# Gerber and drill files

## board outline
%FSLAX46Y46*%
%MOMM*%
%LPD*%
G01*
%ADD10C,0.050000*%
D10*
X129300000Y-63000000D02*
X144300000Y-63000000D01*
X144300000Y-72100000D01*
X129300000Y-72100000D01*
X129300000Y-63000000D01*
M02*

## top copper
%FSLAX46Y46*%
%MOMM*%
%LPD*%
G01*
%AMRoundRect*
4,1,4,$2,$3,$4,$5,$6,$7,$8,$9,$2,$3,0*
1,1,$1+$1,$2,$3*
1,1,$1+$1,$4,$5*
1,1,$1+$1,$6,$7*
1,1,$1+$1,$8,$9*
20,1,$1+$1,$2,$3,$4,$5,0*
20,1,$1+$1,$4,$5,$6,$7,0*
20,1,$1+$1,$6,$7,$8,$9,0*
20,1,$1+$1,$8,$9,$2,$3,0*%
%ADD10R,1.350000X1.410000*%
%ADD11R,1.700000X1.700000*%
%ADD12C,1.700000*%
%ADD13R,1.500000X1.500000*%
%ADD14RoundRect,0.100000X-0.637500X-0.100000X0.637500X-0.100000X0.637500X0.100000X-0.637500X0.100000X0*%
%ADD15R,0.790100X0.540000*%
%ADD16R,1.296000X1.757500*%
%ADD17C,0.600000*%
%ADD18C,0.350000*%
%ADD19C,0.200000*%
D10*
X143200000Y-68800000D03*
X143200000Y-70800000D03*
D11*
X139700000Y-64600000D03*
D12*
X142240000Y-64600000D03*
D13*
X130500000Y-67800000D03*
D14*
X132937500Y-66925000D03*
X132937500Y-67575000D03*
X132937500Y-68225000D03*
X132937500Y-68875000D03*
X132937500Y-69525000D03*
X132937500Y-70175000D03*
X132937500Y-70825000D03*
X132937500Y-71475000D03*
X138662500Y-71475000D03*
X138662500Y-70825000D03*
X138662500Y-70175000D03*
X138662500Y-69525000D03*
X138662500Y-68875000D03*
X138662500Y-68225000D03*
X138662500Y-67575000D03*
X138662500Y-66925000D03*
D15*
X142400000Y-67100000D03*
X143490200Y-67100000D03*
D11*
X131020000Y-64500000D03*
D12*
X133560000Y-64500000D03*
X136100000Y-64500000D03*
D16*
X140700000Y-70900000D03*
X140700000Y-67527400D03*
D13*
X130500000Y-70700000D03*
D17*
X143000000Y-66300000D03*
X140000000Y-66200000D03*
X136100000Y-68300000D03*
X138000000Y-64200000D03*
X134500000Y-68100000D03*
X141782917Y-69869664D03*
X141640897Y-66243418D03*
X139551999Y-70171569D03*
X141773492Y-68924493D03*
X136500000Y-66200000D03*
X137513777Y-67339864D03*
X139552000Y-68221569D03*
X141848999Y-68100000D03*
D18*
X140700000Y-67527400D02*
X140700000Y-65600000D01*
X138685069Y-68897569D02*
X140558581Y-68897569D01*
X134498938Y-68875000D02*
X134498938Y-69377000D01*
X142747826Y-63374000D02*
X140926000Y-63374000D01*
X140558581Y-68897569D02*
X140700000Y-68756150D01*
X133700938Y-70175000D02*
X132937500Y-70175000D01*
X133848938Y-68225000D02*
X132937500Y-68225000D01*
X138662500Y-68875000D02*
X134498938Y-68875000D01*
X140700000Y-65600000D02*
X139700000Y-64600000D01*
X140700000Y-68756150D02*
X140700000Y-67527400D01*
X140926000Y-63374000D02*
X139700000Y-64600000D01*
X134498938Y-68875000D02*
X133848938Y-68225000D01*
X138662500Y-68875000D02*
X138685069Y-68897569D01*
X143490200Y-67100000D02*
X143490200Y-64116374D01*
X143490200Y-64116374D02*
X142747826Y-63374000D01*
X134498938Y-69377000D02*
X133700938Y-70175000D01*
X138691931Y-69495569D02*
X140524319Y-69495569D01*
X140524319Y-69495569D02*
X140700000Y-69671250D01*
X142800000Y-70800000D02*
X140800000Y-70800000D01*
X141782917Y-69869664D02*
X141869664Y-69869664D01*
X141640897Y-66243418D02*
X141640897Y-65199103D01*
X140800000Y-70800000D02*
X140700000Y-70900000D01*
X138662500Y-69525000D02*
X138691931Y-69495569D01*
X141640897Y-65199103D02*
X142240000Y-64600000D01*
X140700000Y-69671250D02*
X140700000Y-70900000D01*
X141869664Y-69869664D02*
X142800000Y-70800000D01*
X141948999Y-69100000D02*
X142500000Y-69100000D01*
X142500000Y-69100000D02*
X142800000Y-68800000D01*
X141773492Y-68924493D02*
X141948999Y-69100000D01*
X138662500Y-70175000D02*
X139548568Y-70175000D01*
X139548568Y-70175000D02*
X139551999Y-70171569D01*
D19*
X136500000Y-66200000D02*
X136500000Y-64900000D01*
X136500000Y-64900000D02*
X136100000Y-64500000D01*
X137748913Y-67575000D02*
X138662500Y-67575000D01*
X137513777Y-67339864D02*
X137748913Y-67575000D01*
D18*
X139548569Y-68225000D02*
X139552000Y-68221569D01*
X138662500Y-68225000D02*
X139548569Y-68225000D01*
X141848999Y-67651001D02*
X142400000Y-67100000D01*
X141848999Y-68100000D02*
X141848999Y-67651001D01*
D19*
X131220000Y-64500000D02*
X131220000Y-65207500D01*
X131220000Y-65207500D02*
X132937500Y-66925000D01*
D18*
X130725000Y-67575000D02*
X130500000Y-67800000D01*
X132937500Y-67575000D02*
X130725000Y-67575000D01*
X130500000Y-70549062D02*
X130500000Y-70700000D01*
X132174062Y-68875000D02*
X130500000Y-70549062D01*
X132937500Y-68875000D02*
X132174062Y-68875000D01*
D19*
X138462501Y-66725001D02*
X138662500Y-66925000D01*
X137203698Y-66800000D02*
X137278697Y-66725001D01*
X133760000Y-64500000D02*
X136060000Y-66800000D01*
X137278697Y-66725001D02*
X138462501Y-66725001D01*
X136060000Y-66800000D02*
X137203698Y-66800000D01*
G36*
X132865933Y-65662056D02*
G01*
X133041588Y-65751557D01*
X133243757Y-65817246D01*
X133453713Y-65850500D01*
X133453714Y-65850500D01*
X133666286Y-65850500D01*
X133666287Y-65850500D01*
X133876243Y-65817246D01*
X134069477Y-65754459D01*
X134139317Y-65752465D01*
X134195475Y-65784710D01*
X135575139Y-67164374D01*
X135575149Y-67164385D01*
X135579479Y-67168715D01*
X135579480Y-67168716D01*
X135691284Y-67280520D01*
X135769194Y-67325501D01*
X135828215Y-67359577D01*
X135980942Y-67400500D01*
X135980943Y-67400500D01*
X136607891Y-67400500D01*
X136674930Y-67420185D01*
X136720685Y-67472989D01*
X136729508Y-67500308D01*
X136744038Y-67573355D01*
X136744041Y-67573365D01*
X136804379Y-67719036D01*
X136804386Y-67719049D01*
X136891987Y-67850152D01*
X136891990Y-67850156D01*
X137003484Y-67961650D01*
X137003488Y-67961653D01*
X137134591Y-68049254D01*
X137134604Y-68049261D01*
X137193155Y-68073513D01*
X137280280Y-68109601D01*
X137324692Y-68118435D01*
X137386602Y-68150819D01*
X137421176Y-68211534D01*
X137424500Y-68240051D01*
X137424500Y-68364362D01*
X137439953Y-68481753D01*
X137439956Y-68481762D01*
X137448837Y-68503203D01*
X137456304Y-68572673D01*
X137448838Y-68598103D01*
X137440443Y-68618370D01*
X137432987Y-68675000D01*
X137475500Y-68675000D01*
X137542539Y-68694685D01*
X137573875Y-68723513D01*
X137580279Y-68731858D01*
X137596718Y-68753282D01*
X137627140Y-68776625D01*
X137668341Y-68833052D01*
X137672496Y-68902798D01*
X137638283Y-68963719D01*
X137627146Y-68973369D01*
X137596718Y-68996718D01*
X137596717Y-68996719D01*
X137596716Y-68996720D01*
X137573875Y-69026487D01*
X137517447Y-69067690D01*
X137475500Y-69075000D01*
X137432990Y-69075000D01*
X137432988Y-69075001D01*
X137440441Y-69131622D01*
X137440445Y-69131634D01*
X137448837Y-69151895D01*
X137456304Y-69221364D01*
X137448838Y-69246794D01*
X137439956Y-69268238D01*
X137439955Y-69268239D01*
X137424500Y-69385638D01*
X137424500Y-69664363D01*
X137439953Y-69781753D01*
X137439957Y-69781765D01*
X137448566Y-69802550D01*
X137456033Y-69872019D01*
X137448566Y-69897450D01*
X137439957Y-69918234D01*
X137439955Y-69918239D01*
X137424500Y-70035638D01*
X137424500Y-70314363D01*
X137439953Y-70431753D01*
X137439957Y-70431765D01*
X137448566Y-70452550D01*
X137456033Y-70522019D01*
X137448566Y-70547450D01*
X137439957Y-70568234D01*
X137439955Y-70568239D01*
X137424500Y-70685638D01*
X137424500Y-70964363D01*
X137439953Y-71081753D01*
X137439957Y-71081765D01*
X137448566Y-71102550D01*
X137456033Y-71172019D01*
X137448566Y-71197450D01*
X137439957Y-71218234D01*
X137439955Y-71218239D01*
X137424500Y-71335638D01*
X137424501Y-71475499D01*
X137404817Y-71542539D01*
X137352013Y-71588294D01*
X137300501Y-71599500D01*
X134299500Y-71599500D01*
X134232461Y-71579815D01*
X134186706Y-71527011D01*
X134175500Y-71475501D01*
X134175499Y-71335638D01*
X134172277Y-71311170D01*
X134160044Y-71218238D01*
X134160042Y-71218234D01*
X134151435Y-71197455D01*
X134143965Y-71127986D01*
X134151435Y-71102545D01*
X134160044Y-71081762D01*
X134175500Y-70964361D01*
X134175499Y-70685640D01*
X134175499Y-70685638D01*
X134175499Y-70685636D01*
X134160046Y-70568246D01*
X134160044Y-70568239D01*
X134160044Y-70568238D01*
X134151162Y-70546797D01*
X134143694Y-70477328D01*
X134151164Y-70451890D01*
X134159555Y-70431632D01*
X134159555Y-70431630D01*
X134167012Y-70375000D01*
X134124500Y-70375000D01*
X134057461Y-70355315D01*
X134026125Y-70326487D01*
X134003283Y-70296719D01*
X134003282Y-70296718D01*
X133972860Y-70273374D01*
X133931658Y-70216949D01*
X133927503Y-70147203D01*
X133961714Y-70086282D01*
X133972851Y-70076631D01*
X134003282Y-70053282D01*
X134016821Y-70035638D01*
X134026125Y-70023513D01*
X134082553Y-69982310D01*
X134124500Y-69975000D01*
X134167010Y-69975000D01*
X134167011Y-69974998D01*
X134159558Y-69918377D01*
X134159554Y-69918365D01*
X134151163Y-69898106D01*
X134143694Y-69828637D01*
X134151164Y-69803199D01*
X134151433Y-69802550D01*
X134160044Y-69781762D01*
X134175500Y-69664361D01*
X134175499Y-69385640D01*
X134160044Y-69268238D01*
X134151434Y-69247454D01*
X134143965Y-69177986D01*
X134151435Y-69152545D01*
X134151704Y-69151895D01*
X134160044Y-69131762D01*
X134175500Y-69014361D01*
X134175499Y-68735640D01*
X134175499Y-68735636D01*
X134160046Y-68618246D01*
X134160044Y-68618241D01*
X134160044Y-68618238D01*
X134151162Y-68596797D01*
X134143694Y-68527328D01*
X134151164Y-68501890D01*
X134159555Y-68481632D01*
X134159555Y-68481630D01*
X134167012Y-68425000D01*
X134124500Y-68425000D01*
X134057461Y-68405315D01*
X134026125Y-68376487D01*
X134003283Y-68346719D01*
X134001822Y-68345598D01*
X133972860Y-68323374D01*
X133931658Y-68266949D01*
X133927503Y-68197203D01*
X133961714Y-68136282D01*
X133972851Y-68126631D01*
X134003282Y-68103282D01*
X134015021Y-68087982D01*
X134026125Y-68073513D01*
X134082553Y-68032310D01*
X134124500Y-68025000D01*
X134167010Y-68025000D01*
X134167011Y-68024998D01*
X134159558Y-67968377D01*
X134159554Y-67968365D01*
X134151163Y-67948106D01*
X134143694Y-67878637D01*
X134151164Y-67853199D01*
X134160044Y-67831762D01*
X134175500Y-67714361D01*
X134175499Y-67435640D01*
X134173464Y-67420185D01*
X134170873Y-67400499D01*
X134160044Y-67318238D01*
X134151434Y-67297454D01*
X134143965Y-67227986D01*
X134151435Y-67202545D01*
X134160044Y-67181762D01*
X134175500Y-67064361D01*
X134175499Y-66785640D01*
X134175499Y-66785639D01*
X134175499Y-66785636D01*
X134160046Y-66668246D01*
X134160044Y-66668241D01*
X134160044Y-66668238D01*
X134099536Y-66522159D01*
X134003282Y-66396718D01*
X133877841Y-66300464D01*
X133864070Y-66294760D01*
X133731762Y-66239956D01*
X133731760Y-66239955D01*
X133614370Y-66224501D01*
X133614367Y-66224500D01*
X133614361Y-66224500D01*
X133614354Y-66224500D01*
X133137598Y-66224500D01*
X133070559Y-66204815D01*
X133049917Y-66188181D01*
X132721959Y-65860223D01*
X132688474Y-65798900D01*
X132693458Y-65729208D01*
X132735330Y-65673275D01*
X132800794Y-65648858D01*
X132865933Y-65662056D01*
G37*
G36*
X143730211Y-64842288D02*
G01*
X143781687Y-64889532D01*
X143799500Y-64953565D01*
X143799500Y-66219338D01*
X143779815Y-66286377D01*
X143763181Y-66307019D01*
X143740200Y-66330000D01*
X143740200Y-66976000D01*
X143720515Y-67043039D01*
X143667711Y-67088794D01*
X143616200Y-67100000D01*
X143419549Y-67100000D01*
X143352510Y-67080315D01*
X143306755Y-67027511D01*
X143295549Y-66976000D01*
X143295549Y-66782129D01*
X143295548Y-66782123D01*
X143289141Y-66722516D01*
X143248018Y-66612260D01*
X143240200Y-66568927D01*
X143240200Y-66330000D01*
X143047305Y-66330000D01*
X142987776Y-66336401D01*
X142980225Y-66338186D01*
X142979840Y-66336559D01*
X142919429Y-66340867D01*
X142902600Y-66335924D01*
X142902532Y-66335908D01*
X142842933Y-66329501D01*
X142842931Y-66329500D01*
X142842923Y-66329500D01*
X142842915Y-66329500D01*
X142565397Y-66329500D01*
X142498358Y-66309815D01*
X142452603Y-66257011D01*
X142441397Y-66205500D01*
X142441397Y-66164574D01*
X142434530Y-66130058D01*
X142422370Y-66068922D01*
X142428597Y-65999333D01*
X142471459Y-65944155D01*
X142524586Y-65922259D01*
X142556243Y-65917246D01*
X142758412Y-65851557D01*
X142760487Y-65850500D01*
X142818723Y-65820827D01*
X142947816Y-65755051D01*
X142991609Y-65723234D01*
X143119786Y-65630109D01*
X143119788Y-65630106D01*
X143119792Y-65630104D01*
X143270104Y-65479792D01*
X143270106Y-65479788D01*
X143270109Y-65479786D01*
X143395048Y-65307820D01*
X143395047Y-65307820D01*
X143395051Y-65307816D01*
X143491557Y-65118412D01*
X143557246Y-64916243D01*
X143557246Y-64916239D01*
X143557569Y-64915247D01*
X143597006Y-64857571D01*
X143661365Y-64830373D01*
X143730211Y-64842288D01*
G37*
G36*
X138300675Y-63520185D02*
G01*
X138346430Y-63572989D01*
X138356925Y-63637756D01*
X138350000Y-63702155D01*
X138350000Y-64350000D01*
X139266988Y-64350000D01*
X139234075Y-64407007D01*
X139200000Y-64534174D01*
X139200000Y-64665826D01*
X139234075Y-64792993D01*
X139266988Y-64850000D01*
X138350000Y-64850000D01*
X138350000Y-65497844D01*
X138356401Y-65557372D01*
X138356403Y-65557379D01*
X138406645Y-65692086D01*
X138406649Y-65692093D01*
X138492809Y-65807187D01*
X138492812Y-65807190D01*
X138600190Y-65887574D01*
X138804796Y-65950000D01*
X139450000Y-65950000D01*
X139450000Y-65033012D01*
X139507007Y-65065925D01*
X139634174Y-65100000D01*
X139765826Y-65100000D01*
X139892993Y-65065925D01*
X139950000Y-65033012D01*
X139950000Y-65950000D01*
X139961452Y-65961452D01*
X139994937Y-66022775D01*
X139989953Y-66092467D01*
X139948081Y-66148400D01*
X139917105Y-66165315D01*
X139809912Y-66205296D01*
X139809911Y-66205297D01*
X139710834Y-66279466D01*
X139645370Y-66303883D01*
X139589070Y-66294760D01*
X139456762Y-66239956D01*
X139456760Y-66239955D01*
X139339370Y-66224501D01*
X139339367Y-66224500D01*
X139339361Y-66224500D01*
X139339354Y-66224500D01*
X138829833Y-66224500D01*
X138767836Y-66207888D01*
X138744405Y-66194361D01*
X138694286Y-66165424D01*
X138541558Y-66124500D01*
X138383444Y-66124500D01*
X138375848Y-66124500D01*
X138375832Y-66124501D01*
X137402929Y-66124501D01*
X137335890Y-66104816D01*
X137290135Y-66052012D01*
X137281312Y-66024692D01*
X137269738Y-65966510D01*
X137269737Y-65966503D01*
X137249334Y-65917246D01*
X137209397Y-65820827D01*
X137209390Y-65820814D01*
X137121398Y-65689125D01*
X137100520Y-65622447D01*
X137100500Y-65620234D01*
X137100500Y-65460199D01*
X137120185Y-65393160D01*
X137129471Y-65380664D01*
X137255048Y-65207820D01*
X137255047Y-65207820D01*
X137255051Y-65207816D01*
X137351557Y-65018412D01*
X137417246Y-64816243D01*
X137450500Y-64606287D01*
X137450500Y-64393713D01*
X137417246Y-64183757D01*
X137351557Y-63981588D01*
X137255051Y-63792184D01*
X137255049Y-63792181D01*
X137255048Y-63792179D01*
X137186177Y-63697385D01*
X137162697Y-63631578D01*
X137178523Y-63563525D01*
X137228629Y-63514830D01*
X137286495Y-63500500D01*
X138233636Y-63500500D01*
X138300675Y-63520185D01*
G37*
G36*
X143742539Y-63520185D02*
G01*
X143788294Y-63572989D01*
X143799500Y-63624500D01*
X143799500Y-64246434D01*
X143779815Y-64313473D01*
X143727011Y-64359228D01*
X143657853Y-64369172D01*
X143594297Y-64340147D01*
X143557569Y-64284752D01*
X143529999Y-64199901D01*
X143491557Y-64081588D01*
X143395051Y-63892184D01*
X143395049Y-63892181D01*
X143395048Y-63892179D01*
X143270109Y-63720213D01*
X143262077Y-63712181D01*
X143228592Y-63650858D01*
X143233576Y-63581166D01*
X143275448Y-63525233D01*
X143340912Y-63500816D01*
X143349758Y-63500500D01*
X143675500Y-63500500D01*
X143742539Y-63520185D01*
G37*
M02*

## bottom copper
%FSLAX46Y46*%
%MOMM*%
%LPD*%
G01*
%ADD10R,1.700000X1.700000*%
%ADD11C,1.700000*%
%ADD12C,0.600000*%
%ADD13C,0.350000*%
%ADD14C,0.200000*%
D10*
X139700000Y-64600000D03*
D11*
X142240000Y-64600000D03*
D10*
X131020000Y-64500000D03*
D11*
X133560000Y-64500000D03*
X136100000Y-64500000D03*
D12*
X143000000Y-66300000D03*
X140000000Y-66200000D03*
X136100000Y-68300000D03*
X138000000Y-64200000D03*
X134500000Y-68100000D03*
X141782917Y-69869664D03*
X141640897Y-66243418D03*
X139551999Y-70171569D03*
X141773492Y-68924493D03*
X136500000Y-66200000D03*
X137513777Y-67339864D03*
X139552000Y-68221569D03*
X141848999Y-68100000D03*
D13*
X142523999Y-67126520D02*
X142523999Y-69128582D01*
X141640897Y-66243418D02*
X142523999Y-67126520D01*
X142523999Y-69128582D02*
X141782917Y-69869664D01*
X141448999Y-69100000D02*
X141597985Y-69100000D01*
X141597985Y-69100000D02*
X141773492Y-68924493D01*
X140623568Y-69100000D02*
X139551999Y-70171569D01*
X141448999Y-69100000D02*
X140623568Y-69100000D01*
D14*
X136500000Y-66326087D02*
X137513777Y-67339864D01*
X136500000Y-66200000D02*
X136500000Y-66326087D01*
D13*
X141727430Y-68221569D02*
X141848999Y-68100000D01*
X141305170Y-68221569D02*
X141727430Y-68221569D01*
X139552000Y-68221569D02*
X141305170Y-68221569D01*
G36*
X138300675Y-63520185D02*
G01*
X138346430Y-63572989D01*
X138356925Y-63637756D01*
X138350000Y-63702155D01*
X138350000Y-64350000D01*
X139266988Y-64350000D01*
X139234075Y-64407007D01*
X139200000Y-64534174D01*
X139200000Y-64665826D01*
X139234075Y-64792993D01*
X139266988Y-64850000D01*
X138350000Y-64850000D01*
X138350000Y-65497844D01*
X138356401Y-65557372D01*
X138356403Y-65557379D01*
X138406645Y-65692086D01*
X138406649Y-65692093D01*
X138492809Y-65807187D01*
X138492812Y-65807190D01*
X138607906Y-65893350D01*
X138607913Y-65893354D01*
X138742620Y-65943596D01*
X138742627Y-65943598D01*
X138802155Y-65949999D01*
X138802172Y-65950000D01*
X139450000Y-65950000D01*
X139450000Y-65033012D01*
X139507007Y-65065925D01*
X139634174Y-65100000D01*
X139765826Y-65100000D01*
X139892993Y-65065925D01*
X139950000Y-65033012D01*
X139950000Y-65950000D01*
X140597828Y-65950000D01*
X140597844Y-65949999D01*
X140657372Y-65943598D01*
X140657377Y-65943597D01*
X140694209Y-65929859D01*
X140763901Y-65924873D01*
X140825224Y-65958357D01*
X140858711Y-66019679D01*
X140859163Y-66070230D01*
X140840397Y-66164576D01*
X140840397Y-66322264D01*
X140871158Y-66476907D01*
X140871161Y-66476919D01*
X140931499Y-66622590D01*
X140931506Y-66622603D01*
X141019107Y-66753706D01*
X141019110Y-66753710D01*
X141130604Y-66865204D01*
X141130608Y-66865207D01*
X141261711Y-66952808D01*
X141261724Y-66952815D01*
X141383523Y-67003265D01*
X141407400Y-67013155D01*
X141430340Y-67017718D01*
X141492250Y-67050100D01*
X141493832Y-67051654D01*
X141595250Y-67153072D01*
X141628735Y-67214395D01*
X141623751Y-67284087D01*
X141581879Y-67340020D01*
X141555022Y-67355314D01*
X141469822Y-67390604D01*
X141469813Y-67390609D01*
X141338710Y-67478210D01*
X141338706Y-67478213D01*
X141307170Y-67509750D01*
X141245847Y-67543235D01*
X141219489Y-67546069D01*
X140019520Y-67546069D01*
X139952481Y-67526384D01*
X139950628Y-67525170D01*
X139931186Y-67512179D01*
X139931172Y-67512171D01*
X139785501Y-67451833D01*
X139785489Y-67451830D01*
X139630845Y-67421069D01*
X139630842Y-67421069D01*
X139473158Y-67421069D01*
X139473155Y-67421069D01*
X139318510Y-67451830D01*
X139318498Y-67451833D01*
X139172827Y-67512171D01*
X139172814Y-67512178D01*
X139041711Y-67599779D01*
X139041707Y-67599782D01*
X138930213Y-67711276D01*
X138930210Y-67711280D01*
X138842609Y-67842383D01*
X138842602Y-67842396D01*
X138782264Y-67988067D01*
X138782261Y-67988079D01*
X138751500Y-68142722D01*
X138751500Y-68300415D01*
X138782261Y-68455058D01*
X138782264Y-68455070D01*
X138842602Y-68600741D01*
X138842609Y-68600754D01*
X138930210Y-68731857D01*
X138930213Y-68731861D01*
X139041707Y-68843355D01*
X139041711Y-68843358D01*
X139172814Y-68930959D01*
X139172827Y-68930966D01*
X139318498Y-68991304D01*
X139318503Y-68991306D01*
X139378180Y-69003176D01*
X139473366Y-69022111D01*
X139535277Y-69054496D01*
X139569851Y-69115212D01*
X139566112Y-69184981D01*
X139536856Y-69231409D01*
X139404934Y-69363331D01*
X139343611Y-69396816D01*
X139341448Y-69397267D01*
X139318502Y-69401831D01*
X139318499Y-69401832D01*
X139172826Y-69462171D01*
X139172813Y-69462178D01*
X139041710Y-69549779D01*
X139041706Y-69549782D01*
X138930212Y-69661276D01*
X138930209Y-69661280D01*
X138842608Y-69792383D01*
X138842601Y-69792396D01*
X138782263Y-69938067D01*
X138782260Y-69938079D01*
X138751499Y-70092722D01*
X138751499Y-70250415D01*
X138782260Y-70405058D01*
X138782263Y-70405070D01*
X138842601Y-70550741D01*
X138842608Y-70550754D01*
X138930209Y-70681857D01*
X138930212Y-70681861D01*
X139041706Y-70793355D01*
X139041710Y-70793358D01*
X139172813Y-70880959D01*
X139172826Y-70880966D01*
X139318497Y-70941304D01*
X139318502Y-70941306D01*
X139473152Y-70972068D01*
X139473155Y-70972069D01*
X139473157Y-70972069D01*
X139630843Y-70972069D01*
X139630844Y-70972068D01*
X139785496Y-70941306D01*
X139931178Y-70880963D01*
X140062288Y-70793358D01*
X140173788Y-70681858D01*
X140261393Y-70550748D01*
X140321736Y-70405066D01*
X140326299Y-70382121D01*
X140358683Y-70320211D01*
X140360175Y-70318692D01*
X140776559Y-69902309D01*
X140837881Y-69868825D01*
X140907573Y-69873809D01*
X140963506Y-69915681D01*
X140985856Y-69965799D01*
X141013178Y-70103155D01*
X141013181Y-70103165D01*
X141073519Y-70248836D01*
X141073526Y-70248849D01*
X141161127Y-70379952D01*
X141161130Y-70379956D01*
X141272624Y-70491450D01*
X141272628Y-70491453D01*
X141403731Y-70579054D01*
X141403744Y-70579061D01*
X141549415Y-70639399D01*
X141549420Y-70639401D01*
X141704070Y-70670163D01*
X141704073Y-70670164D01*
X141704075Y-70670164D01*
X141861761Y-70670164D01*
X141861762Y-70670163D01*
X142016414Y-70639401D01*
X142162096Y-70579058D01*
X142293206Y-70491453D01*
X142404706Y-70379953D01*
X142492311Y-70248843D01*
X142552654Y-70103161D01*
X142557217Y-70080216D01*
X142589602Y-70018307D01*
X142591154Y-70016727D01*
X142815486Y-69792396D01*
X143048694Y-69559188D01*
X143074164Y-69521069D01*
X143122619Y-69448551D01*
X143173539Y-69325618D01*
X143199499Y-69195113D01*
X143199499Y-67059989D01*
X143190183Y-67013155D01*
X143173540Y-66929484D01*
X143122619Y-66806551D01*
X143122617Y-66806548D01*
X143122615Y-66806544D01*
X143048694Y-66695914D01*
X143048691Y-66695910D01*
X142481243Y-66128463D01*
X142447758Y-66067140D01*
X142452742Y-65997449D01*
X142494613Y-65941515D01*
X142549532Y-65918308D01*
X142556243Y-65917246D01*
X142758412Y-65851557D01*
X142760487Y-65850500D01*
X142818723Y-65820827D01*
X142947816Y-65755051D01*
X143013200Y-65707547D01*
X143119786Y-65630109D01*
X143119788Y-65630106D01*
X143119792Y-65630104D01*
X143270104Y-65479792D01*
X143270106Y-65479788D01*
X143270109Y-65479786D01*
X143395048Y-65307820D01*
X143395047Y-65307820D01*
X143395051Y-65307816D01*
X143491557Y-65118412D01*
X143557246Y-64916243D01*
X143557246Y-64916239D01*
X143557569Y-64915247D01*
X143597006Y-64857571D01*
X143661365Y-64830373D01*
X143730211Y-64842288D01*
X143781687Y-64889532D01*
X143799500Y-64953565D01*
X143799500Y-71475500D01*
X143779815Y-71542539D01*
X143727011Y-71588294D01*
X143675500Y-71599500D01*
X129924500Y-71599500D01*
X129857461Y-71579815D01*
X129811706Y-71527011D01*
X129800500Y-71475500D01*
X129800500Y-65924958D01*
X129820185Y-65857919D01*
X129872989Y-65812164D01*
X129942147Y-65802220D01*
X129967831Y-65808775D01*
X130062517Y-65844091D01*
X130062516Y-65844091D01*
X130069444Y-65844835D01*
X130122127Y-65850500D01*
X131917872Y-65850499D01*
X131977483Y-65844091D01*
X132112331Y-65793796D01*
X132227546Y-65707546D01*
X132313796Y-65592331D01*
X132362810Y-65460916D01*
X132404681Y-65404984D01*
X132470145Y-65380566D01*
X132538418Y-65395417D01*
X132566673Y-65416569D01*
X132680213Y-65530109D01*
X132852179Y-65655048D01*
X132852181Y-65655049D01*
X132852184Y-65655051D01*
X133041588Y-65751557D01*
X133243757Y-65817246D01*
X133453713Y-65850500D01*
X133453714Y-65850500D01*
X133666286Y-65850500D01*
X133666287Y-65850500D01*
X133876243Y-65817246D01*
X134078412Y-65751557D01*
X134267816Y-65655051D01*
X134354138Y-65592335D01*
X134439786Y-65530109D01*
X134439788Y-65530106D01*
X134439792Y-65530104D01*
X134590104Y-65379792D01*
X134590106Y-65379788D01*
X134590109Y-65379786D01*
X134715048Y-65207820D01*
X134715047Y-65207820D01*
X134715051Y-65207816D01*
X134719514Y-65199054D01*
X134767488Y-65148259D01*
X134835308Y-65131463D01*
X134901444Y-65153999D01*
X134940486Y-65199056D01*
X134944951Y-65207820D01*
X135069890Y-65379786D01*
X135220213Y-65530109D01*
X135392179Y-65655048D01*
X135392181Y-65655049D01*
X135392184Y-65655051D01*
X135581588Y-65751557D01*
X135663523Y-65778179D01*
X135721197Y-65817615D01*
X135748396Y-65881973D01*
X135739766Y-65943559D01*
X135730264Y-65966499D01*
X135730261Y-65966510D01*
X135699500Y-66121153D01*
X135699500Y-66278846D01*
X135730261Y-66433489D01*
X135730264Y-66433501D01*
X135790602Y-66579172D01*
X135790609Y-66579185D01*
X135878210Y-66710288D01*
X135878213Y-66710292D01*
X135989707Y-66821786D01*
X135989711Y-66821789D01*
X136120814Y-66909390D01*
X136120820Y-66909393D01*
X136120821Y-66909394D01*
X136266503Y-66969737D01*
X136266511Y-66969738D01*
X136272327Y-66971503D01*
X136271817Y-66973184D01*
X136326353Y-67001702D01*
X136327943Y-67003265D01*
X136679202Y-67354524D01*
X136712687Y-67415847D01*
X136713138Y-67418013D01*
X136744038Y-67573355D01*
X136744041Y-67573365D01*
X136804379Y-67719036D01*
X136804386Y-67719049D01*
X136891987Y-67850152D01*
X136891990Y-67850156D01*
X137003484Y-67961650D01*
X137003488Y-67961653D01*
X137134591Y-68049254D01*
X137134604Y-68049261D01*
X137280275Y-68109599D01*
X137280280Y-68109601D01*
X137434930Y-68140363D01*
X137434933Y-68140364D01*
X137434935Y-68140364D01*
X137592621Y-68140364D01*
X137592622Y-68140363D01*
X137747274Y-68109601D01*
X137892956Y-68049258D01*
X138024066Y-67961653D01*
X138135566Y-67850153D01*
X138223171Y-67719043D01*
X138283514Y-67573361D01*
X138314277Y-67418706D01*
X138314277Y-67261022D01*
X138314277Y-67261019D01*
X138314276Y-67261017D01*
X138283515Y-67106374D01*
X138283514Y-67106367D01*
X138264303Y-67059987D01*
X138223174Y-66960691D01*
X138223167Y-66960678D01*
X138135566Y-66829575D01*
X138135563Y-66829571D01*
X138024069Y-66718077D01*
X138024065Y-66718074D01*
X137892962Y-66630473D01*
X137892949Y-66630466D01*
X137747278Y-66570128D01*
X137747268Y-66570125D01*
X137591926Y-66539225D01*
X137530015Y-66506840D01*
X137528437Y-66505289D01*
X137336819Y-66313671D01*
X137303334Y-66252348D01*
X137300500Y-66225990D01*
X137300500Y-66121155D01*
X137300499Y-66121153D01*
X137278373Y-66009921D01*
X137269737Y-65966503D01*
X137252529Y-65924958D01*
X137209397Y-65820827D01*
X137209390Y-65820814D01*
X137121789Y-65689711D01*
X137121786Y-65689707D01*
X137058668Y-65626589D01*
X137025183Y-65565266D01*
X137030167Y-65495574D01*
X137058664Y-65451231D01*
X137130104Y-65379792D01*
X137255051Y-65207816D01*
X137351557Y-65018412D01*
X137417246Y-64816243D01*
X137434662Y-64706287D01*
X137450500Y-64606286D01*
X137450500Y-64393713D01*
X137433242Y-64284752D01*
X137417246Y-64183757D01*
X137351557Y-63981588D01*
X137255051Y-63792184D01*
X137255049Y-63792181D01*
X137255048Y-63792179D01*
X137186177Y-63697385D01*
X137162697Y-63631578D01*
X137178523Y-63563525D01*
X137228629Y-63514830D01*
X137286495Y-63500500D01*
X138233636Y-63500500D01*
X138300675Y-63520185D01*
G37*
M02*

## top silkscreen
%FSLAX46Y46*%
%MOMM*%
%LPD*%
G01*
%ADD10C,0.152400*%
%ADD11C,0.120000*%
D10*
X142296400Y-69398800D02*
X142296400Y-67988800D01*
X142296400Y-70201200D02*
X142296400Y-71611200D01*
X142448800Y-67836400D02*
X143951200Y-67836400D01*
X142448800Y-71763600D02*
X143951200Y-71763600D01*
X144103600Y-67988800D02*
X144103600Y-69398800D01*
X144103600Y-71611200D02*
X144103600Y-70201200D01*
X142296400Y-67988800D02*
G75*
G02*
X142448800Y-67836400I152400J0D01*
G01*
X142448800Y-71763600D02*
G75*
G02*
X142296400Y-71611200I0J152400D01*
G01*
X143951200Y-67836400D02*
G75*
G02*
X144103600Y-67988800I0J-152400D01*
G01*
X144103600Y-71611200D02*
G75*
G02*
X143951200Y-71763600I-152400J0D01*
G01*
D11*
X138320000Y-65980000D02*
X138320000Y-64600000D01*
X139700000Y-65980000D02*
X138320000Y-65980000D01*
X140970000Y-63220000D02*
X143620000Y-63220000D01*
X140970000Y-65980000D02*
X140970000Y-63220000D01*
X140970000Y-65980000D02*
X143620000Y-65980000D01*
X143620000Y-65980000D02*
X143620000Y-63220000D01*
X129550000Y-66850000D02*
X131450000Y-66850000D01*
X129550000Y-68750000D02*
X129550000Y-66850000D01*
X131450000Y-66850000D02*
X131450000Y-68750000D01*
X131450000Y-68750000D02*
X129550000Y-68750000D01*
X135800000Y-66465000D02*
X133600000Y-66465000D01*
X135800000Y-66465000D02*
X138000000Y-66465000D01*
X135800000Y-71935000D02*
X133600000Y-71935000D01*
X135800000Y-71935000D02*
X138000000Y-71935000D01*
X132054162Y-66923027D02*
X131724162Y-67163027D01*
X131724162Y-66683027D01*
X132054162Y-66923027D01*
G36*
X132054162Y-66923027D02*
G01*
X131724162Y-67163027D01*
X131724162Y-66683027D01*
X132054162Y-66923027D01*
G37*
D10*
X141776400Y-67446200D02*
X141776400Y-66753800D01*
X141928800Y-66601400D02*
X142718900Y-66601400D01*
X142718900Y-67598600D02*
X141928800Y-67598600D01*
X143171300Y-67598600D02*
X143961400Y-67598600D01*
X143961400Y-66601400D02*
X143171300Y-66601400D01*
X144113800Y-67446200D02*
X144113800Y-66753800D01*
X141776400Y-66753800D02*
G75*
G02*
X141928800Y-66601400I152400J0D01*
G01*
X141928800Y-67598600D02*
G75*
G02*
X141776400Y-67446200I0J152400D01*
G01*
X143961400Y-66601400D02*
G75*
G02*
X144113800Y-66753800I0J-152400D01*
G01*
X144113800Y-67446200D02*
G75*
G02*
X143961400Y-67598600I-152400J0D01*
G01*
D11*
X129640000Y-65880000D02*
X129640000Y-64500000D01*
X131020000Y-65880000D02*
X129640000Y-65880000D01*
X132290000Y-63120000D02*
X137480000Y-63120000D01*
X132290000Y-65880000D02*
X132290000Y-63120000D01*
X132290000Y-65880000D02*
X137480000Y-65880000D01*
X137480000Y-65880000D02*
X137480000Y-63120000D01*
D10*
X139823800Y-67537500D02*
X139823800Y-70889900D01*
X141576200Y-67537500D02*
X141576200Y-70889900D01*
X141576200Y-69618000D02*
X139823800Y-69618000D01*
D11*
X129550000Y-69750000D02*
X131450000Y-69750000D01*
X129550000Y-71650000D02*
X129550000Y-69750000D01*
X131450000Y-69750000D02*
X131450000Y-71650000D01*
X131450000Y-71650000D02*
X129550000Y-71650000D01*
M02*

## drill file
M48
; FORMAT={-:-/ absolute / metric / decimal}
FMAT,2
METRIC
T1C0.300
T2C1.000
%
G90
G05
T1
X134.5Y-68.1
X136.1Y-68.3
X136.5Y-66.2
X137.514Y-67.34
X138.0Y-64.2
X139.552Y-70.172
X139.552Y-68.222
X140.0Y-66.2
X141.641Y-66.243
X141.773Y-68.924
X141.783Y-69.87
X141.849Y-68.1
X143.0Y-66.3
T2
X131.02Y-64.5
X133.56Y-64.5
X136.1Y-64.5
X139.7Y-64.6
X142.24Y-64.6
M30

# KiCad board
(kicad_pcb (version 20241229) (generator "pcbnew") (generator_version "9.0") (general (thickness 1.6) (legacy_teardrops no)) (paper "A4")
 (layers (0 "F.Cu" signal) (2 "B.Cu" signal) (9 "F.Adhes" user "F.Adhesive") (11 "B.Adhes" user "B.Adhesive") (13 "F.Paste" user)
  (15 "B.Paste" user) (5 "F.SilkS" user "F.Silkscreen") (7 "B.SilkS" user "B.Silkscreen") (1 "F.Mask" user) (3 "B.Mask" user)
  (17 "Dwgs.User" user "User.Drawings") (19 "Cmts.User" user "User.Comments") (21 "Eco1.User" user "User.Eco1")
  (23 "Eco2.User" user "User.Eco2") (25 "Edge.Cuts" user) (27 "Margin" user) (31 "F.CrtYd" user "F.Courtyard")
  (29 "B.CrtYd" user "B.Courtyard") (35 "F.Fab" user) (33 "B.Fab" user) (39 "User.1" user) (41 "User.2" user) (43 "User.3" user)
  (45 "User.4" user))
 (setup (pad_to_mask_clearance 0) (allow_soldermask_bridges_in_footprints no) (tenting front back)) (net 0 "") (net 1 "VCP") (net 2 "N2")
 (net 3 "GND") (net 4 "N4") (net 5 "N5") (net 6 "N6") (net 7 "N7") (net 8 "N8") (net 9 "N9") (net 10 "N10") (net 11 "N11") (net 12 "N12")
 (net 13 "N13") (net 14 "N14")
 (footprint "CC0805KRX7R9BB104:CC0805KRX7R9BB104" (layer "F.Cu") (at 143.2 69.8 -90)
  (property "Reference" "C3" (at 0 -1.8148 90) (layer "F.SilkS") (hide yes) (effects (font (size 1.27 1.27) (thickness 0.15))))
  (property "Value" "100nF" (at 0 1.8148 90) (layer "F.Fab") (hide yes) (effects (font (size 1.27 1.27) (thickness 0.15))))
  (fp_line (start -0.4012 0.9036) (end -1.8112 0.9036) (stroke (width 0.1524) (type default)) (layer "F.SilkS"))
  (fp_line (start 0.4012 0.9036) (end 1.8112 0.9036) (stroke (width 0.1524) (type default)) (layer "F.SilkS"))
  (fp_line (start -1.9636 0.7512) (end -1.9636 -0.7512) (stroke (width 0.1524) (type default)) (layer "F.SilkS"))
  (fp_line (start 1.9636 0.7512) (end 1.9636 -0.7512) (stroke (width 0.1524) (type default)) (layer "F.SilkS"))
  (fp_line (start -1.8112 -0.9036) (end -0.4012 -0.9036) (stroke (width 0.1524) (type default)) (layer "F.SilkS"))
  (fp_line (start 1.8112 -0.9036) (end 0.4012 -0.9036) (stroke (width 0.1524) (type default)) (layer "F.SilkS"))
  (fp_arc (start -1.8112 0.9036) (mid -1.918963 0.858963) (end -1.9636 0.7512) (stroke (width 0.1524) (type default)) (layer "F.SilkS"))
  (fp_arc (start 1.9636 0.7512) (mid 1.918963 0.858963) (end 1.8112 0.9036) (stroke (width 0.1524) (type default)) (layer "F.SilkS"))
  (fp_arc (start -1.9636 -0.7512) (mid -1.918963 -0.858963) (end -1.8112 -0.9036) (stroke (width 0.1524) (type default)) (layer "F.SilkS"))
  (fp_arc (start 1.8112 -0.9036) (mid 1.918963 -0.858963) (end 1.9636 -0.7512) (stroke (width 0.1524) (type default)) (layer "F.SilkS"))
  (pad "1" smd rect (at -1 0 270) (size 1.41 1.35) (layers "F.Cu" "F.Mask" "F.Paste") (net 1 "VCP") (solder_mask_margin 0.0508)
   (solder_paste_margin -100) (thermal_bridge_angle 0))
  (pad "2" smd rect (at 1 0 270) (size 1.41 1.35) (layers "F.Cu" "F.Mask" "F.Paste") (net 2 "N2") (solder_mask_margin 0.0508)
   (solder_paste_margin -100) (thermal_bridge_angle 0))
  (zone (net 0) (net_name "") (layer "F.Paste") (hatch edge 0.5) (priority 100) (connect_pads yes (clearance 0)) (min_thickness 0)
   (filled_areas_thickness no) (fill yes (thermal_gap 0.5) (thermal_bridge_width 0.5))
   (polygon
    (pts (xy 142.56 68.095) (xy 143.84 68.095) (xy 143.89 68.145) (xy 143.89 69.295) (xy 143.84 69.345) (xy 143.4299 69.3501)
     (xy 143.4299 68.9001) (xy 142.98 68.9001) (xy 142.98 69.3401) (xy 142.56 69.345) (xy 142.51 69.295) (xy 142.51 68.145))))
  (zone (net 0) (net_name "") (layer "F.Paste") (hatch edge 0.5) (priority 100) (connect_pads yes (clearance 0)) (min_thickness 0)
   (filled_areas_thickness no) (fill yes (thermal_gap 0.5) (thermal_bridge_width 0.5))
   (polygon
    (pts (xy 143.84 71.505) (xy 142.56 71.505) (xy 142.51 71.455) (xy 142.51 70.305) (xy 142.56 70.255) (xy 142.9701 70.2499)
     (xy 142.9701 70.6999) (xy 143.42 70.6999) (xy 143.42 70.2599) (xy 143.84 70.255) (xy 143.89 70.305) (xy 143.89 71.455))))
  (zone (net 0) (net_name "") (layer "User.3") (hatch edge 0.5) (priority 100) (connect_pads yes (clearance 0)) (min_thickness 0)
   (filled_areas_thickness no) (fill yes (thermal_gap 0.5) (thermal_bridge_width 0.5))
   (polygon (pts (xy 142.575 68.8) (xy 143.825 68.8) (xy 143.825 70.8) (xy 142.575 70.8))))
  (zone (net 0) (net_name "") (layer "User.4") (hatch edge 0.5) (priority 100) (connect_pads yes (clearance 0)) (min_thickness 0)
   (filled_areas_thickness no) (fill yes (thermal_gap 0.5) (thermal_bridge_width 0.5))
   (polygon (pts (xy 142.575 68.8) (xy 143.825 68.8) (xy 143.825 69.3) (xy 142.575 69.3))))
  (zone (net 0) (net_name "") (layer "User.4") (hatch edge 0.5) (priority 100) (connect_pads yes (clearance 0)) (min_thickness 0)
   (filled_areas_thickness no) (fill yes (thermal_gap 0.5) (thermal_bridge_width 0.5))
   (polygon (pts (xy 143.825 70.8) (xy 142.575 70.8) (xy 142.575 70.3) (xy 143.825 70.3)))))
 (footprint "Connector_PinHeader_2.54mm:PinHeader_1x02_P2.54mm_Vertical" (layer "F.Cu") (at 139.7 64.6 90)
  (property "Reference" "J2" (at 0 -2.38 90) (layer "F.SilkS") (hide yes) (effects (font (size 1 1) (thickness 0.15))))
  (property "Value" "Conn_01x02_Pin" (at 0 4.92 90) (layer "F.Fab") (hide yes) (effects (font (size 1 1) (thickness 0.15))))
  (fp_line (start -1.38 -1.38) (end 0 -1.38) (stroke (width 0.12) (type solid)) (layer "F.SilkS"))
  (fp_line (start -1.38 0) (end -1.38 -1.38) (stroke (width 0.12) (type solid)) (layer "F.SilkS"))
  (fp_line (start 1.38 1.27) (end 1.38 3.92) (stroke (width 0.12) (type solid)) (layer "F.SilkS"))
  (fp_line (start -1.38 1.27) (end 1.38 1.27) (stroke (width 0.12) (type solid)) (layer "F.SilkS"))
  (fp_line (start -1.38 1.27) (end -1.38 3.92) (stroke (width 0.12) (type solid)) (layer "F.SilkS"))
  (fp_line (start -1.38 3.92) (end 1.38 3.92) (stroke (width 0.12) (type solid)) (layer "F.SilkS"))
  (pad "1" thru_hole rect (at 0 0 90) (size 1.7 1.7) (drill 1) (layers "*.Cu" "*.Mask") (remove_unused_layers no) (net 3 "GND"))
  (pad "2" thru_hole circle (at 0 2.54 90) (size 1.7 1.7) (drill 1) (layers "*.Cu" "*.Mask") (remove_unused_layers no) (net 2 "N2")))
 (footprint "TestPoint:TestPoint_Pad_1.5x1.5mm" (layer "F.Cu") (at 130.5 67.8)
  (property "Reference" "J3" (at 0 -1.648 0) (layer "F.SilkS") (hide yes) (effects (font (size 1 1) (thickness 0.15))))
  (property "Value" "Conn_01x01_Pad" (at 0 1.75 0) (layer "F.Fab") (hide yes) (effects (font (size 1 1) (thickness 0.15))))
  (fp_line (start -0.95 -0.95) (end 0.95 -0.95) (stroke (width 0.12) (type solid)) (layer "F.SilkS"))
  (fp_line (start -0.95 0.95) (end -0.95 -0.95) (stroke (width 0.12) (type solid)) (layer "F.SilkS"))
  (fp_line (start 0.95 -0.95) (end 0.95 0.95) (stroke (width 0.12) (type solid)) (layer "F.SilkS"))
  (fp_line (start 0.95 0.95) (end -0.95 0.95) (stroke (width 0.12) (type solid)) (layer "F.SilkS"))
  (pad "1" smd rect (at 0 0) (size 1.5 1.5) (layers "F.Cu" "F.Mask") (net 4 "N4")))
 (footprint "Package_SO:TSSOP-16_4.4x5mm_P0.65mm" (layer "F.Cu") (at 135.8 69.2)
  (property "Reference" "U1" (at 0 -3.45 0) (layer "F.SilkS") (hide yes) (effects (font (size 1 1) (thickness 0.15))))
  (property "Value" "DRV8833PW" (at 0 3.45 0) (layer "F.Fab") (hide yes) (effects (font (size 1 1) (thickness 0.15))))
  (fp_line (start 0 -2.735) (end -2.2 -2.735) (stroke (width 0.12) (type solid)) (layer "F.SilkS"))
  (fp_line (start 0 -2.735) (end 2.2 -2.735) (stroke (width 0.12) (type solid)) (layer "F.SilkS"))
  (fp_line (start 0 2.735) (end -2.2 2.735) (stroke (width 0.12) (type solid)) (layer "F.SilkS"))
  (fp_line (start 0 2.735) (end 2.2 2.735) (stroke (width 0.12) (type solid)) (layer "F.SilkS"))
  (fp_poly
   (pts (xy -3.745838 -2.276973) (xy -4.075838 -2.036973) (xy -4.075838 -2.516973)) (stroke (width 0.12) (type solid)) (fill yes)
   (layer "F.SilkS"))
  (pad "1" smd roundrect (at -2.8625 -2.275) (size 1.475 0.4) (layers "F.Cu" "F.Mask" "F.Paste") (roundrect_rratio 0.25) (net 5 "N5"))
  (pad "2" smd roundrect (at -2.8625 -1.625) (size 1.475 0.4) (layers "F.Cu" "F.Mask" "F.Paste") (roundrect_rratio 0.25) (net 4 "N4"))
  (pad "3" smd roundrect (at -2.8625 -0.975) (size 1.475 0.4) (layers "F.Cu" "F.Mask" "F.Paste") (roundrect_rratio 0.25) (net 3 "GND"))
  (pad "4" smd roundrect (at -2.8625 -0.325) (size 1.475 0.4) (layers "F.Cu" "F.Mask" "F.Paste") (roundrect_rratio 0.25) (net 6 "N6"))
  (pad "5" smd roundrect (at -2.8625 0.325) (size 1.475 0.4) (layers "F.Cu" "F.Mask" "F.Paste") (roundrect_rratio 0.25) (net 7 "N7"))
  (pad "6" smd roundrect (at -2.8625 0.975) (size 1.475 0.4) (layers "F.Cu" "F.Mask" "F.Paste") (roundrect_rratio 0.25) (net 3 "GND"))
  (pad "7" smd roundrect (at -2.8625 1.625) (size 1.475 0.4) (layers "F.Cu" "F.Mask" "F.Paste") (roundrect_rratio 0.25) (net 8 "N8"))
  (pad "8" smd roundrect (at -2.8625 2.275) (size 1.475 0.4) (layers "F.Cu" "F.Mask" "F.Paste") (roundrect_rratio 0.25) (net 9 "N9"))
  (pad "9" smd roundrect (at 2.8625 2.275) (size 1.475 0.4) (layers "F.Cu" "F.Mask" "F.Paste") (roundrect_rratio 0.25) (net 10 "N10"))
  (pad "10" smd roundrect (at 2.8625 1.625) (size 1.475 0.4) (layers "F.Cu" "F.Mask" "F.Paste") (roundrect_rratio 0.25) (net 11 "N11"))
  (pad "11" smd roundrect (at 2.8625 0.975) (size 1.475 0.4) (layers "F.Cu" "F.Mask" "F.Paste") (roundrect_rratio 0.25) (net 1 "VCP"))
  (pad "12" smd roundrect (at 2.8625 0.325) (size 1.475 0.4) (layers "F.Cu" "F.Mask" "F.Paste") (roundrect_rratio 0.25) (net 2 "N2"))
  (pad "13" smd roundrect (at 2.8625 -0.325) (size 1.475 0.4) (layers "F.Cu" "F.Mask" "F.Paste") (roundrect_rratio 0.25) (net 3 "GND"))
  (pad "14" smd roundrect (at 2.8625 -0.975) (size 1.475 0.4) (layers "F.Cu" "F.Mask" "F.Paste") (roundrect_rratio 0.25) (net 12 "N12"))
  (pad "15" smd roundrect (at 2.8625 -1.625) (size 1.475 0.4) (layers "F.Cu" "F.Mask" "F.Paste") (roundrect_rratio 0.25) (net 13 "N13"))
  (pad "16" smd roundrect (at 2.8625 -2.275) (size 1.475 0.4) (layers "F.Cu" "F.Mask" "F.Paste") (roundrect_rratio 0.25) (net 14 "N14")))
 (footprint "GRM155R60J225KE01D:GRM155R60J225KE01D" (layer "F.Cu") (at 142.9451 67.1)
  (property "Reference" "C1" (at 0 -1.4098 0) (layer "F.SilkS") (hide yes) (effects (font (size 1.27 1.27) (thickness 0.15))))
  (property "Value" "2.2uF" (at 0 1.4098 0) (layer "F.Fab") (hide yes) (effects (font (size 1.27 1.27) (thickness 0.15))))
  (fp_line (start -1.1687 0.3462) (end -1.1687 -0.3462) (stroke (width 0.1524) (type default)) (layer "F.SilkS"))
  (fp_line (start -1.0163 -0.4986) (end -0.2262 -0.4986) (stroke (width 0.1524) (type default)) (layer "F.SilkS"))
  (fp_line (start -0.2262 0.4986) (end -1.0163 0.4986) (stroke (width 0.1524) (type default)) (layer "F.SilkS"))
  (fp_line (start 0.2262 0.4986) (end 1.0163 0.4986) (stroke (width 0.1524) (type default)) (layer "F.SilkS"))
  (fp_line (start 1.0163 -0.4986) (end 0.2262 -0.4986) (stroke (width 0.1524) (type default)) (layer "F.SilkS"))
  (fp_line (start 1.1687 0.3462) (end 1.1687 -0.3462) (stroke (width 0.1524) (type default)) (layer "F.SilkS"))
  (fp_arc (start -1.1687 -0.3462) (mid -1.124063 -0.453963) (end -1.0163 -0.4986) (stroke (width 0.1524) (type default)) (layer "F.SilkS"))
  (fp_arc (start -1.0163 0.4986) (mid -1.124063 0.453963) (end -1.1687 0.3462) (stroke (width 0.1524) (type default)) (layer "F.SilkS"))
  (fp_arc (start 1.0163 -0.4986) (mid 1.124063 -0.453963) (end 1.1687 -0.3462) (stroke (width 0.1524) (type default)) (layer "F.SilkS"))
  (fp_arc (start 1.1687 0.3462) (mid 1.124063 0.453963) (end 1.0163 0.4986) (stroke (width 0.1524) (type default)) (layer "F.SilkS"))
  (pad "1" smd rect (at -0.5451 0) (size 0.7901 0.54) (layers "F.Cu" "F.Mask" "F.Paste") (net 12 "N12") (solder_mask_margin 0.0508)
   (solder_paste_margin -100) (thermal_bridge_angle 0))
  (pad "2" smd rect (at 0.5451 0) (size 0.7901 0.54) (layers "F.Cu" "F.Mask" "F.Paste") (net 3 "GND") (solder_mask_margin 0.0508)
   (solder_paste_margin -100) (thermal_bridge_angle 0))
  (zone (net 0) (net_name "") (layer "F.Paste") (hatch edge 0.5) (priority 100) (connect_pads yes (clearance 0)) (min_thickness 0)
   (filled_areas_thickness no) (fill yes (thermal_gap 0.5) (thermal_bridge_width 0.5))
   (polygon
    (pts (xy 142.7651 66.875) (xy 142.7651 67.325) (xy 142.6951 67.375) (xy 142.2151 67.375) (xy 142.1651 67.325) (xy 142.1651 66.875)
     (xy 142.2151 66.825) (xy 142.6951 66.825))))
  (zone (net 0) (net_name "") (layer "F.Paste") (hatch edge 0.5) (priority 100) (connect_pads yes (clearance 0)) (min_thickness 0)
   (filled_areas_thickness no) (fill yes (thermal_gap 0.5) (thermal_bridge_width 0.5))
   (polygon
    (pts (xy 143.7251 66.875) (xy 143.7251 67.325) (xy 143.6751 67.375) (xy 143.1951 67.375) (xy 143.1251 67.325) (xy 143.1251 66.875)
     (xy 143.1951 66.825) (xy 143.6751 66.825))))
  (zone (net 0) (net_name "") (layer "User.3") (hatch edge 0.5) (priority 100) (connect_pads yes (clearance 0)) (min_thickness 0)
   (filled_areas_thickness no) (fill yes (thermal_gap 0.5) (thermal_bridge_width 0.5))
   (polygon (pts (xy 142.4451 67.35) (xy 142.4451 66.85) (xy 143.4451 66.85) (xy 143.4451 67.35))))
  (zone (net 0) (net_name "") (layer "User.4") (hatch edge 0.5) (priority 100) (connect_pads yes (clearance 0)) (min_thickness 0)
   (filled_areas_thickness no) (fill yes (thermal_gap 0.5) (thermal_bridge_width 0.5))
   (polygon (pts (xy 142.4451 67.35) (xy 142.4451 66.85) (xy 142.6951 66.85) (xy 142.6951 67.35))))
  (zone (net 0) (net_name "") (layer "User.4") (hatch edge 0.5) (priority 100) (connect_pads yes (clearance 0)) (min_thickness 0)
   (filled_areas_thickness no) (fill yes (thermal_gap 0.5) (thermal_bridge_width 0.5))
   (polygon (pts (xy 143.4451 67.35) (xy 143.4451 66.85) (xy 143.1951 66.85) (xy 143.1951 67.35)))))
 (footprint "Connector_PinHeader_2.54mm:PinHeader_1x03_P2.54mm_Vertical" (layer "F.Cu") (at 131.02 64.5 90)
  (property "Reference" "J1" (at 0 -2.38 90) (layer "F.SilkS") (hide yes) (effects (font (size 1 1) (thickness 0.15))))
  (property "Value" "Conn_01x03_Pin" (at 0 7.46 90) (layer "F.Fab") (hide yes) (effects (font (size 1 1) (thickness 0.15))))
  (fp_line (start -1.38 -1.38) (end 0 -1.38) (stroke (width 0.12) (type solid)) (layer "F.SilkS"))
  (fp_line (start -1.38 0) (end -1.38 -1.38) (stroke (width 0.12) (type solid)) (layer "F.SilkS"))
  (fp_line (start 1.38 1.27) (end 1.38 6.46) (stroke (width 0.12) (type solid)) (layer "F.SilkS"))
  (fp_line (start -1.38 1.27) (end 1.38 1.27) (stroke (width 0.12) (type solid)) (layer "F.SilkS"))
  (fp_line (start -1.38 1.27) (end -1.38 6.46) (stroke (width 0.12) (type solid)) (layer "F.SilkS"))
  (fp_line (start -1.38 6.46) (end 1.38 6.46) (stroke (width 0.12) (type solid)) (layer "F.SilkS"))
  (pad "1" thru_hole rect (at 0 0 90) (size 1.7 1.7) (drill 1) (layers "*.Cu" "*.Mask") (remove_unused_layers no) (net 5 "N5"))
  (pad "2" thru_hole circle (at 0 2.54 90) (size 1.7 1.7) (drill 1) (layers "*.Cu" "*.Mask") (remove_unused_layers no) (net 14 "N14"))
  (pad "3" thru_hole circle (at 0 5.08 90) (size 1.7 1.7) (drill 1) (layers "*.Cu" "*.Mask") (remove_unused_layers no) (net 13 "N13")))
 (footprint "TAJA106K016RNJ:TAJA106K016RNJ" (layer "F.Cu") (at 140.7 69.2137 90)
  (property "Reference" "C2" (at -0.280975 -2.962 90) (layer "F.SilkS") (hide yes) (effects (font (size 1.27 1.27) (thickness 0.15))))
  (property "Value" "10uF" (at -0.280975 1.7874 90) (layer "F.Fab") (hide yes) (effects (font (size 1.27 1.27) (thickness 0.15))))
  (fp_line (start 1.6762 -0.8762) (end -1.6762 -0.8762) (stroke (width 0.1524) (type default)) (layer "F.SilkS"))
  (fp_line (start 1.6762 0.8762) (end -1.6762 0.8762) (stroke (width 0.1524) (type default)) (layer "F.SilkS"))
  (fp_line (start -0.4043 0.8762) (end -0.4043 -0.8762) (stroke (width 0.1524) (type default)) (layer "F.SilkS"))
  (pad "1" smd rect (at -1.6863 0 270) (size 1.7575 1.296) (layers "F.Cu" "F.Mask" "F.Paste") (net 2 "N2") (solder_mask_margin 0.0508)
   (solder_paste_margin 0) (thermal_bridge_angle 0))
  (pad "2" smd rect (at 1.6863 0 270) (size 1.7575 1.296) (layers "F.Cu" "F.Mask" "F.Paste") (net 3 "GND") (solder_mask_margin 0.0508)
   (solder_paste_margin 0) (thermal_bridge_angle 0))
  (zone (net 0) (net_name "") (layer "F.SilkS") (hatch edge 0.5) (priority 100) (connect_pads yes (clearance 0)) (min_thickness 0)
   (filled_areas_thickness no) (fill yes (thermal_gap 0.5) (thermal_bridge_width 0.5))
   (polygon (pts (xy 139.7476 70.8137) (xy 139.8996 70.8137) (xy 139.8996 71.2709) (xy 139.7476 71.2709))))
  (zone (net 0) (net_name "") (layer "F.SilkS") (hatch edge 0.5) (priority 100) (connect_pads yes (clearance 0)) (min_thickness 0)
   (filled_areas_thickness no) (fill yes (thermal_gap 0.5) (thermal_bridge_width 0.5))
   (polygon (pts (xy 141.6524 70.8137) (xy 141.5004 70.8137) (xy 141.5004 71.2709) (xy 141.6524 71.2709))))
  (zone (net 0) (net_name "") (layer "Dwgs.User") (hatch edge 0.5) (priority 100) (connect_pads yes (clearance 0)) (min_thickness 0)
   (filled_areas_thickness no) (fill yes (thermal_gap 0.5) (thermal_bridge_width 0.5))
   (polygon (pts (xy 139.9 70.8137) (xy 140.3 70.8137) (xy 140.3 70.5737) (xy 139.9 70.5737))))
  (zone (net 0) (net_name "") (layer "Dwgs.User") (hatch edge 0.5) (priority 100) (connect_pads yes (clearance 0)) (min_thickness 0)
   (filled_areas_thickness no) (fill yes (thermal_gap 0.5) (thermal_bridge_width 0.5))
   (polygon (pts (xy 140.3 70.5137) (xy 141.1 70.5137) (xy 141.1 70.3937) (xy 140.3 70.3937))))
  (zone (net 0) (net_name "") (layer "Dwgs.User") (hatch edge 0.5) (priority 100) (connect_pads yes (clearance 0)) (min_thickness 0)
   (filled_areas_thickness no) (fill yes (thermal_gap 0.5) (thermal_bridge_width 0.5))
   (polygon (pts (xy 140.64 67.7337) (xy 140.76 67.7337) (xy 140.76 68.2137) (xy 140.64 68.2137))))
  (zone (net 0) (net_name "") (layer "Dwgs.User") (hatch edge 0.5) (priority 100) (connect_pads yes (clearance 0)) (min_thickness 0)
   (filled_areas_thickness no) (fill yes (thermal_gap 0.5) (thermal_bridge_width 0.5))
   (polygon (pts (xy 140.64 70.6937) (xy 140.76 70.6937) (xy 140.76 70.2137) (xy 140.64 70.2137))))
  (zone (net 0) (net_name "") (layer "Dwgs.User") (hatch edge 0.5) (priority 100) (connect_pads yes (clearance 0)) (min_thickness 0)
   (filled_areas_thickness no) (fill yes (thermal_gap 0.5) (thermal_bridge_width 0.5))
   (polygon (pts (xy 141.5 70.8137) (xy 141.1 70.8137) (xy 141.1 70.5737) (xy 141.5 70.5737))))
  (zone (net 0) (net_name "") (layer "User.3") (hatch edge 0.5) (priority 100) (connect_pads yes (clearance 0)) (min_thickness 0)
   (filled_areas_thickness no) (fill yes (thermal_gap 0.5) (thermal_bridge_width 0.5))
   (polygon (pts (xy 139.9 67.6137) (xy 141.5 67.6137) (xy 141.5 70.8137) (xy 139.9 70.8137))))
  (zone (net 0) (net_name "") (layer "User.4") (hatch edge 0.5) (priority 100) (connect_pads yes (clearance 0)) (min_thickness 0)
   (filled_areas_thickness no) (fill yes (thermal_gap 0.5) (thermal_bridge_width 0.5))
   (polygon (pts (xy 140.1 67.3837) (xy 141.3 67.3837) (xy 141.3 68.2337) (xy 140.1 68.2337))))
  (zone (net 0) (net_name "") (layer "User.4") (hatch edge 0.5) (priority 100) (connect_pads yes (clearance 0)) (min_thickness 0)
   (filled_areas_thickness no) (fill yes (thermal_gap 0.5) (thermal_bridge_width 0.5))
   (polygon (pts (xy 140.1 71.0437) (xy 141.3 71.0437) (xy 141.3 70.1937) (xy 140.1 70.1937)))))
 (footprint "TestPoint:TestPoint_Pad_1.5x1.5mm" (layer "F.Cu") (at 130.5 70.7)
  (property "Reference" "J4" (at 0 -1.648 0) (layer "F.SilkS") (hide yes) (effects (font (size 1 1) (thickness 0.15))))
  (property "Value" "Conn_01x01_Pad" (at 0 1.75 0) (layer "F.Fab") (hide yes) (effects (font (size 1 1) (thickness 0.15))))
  (fp_line (start -0.95 -0.95) (end 0.95 -0.95) (stroke (width 0.12) (type solid)) (layer "F.SilkS"))
  (fp_line (start -0.95 0.95) (end -0.95 -0.95) (stroke (width 0.12) (type solid)) (layer "F.SilkS"))
  (fp_line (start 0.95 -0.95) (end 0.95 0.95) (stroke (width 0.12) (type solid)) (layer "F.SilkS"))
  (fp_line (start 0.95 0.95) (end -0.95 0.95) (stroke (width 0.12) (type solid)) (layer "F.SilkS"))
  (pad "1" smd rect (at 0 0) (size 1.5 1.5) (layers "F.Cu" "F.Mask") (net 6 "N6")))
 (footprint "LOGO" (layer "B.Cu") (at 130.7 70.3 180)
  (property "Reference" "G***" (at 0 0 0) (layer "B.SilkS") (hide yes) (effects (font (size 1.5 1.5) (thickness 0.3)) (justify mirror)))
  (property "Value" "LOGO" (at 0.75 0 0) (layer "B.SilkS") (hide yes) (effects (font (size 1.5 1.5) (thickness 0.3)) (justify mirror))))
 (gr_rect (start 129.3 63) (end 144.3 72.1) (stroke (width 0.05) (type solid)) (fill no) (layer "Edge.Cuts"))
 (segment (start 140.7 67.5274) (end 140.7 65.6) (width 0.35) (layer "F.Cu") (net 3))
 (segment (start 138.685069 68.897569) (end 140.558581 68.897569) (width 0.35) (layer "F.Cu") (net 3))
 (segment (start 134.498938 68.875) (end 134.498938 69.377) (width 0.35) (layer "F.Cu") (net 3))
 (segment (start 142.747826 63.374) (end 140.926 63.374) (width 0.35) (layer "F.Cu") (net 3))
 (segment (start 140.558581 68.897569) (end 140.7 68.75615) (width 0.35) (layer "F.Cu") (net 3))
 (segment (start 133.700938 70.175) (end 132.9375 70.175) (width 0.35) (layer "F.Cu") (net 3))
 (segment (start 133.848938 68.225) (end 132.9375 68.225) (width 0.35) (layer "F.Cu") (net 3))
 (segment (start 138.6625 68.875) (end 134.498938 68.875) (width 0.35) (layer "F.Cu") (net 3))
 (segment (start 140.7 65.6) (end 139.7 64.6) (width 0.35) (layer "F.Cu") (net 3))
 (segment (start 140.7 68.75615) (end 140.7 67.5274) (width 0.35) (layer "F.Cu") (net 3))
 (segment (start 140.926 63.374) (end 139.7 64.6) (width 0.35) (layer "F.Cu") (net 3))
 (segment (start 134.498938 68.875) (end 133.848938 68.225) (width 0.35) (layer "F.Cu") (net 3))
 (segment (start 138.6625 68.875) (end 138.685069 68.897569) (width 0.35) (layer "F.Cu") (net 3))
 (segment (start 143.4902 67.1) (end 143.4902 64.116374) (width 0.35) (layer "F.Cu") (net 3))
 (segment (start 143.4902 64.116374) (end 142.747826 63.374) (width 0.35) (layer "F.Cu") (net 3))
 (segment (start 134.498938 69.377) (end 133.700938 70.175) (width 0.35) (layer "F.Cu") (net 3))
 (via (at 143 66.3) (size 0.6) (drill 0.3) (layers "F.Cu" "B.Cu") (free yes) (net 3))
 (via (at 140 66.2) (size 0.6) (drill 0.3) (layers "F.Cu" "B.Cu") (free yes) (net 3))
 (via (at 136.1 68.3) (size 0.6) (drill 0.3) (layers "F.Cu" "B.Cu") (free yes) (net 3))
 (via (at 138 64.2) (size 0.6) (drill 0.3) (layers "F.Cu" "B.Cu") (free yes) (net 3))
 (via (at 134.5 68.1) (size 0.6) (drill 0.3) (layers "F.Cu" "B.Cu") (free yes) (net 3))
 (segment (start 138.691931 69.495569) (end 140.524319 69.495569) (width 0.35) (layer "F.Cu") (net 2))
 (segment (start 140.524319 69.495569) (end 140.7 69.67125) (width 0.35) (layer "F.Cu") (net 2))
 (segment (start 142.8 70.8) (end 140.8 70.8) (width 0.35) (layer "F.Cu") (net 2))
 (segment (start 141.782917 69.869664) (end 141.869664 69.869664) (width 0.35) (layer "F.Cu") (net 2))
 (segment (start 141.640897 66.243418) (end 141.640897 65.199103) (width 0.35) (layer "F.Cu") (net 2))
 (segment (start 140.8 70.8) (end 140.7 70.9) (width 0.35) (layer "F.Cu") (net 2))
 (segment (start 138.6625 69.525) (end 138.691931 69.495569) (width 0.35) (layer "F.Cu") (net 2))
 (segment (start 141.640897 65.199103) (end 142.24 64.6) (width 0.35) (layer "F.Cu") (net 2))
 (segment (start 140.7 69.67125) (end 140.7 70.9) (width 0.35) (layer "F.Cu") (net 2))
 (segment (start 141.869664 69.869664) (end 142.8 70.8) (width 0.35) (layer "F.Cu") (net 2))
 (via (at 141.782917 69.869664) (size 0.6) (drill 0.3) (layers "F.Cu" "B.Cu") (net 2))
 (via (at 141.640897 66.243418) (size 0.6) (drill 0.3) (layers "F.Cu" "B.Cu") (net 2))
 (segment (start 142.523999 67.12652) (end 142.523999 69.128582) (width 0.35) (layer "B.Cu") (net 2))
 (segment (start 141.640897 66.243418) (end 142.523999 67.12652) (width 0.35) (layer "B.Cu") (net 2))
 (segment (start 142.523999 69.128582) (end 141.782917 69.869664) (width 0.35) (layer "B.Cu") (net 2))
 (segment (start 141.948999 69.1) (end 142.5 69.1) (width 0.35) (layer "F.Cu") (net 1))
 (segment (start 142.5 69.1) (end 142.8 68.8) (width 0.35) (layer "F.Cu") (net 1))
 (segment (start 141.773492 68.924493) (end 141.948999 69.1) (width 0.35) (layer "F.Cu") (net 1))
 (segment (start 138.6625 70.175) (end 139.548568 70.175) (width 0.35) (layer "F.Cu") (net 1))
 (segment (start 139.548568 70.175) (end 139.551999 70.171569) (width 0.35) (layer "F.Cu") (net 1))
 (via (at 139.551999 70.171569) (size 0.6) (drill 0.3) (layers "F.Cu" "B.Cu") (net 1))
 (via (at 141.773492 68.924493) (size 0.6) (drill 0.3) (layers "F.Cu" "B.Cu") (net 1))
 (segment (start 141.448999 69.1) (end 141.597985 69.1) (width 0.35) (layer "B.Cu") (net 1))
 (segment (start 141.597985 69.1) (end 141.773492 68.924493) (width 0.35) (layer "B.Cu") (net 1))
 (segment (start 140.623568 69.1) (end 139.551999 70.171569) (width 0.35) (layer "B.Cu") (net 1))
 (segment (start 141.448999 69.1) (end 140.623568 69.1) (width 0.35) (layer "B.Cu") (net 1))
 (segment (start 136.5 66.2) (end 136.5 64.9) (width 0.2) (layer "F.Cu") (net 13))
 (segment (start 136.5 64.9) (end 136.1 64.5) (width 0.2) (layer "F.Cu") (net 13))
 (segment (start 137.748913 67.575) (end 138.6625 67.575) (width 0.2) (layer "F.Cu") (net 13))
 (segment (start 137.513777 67.339864) (end 137.748913 67.575) (width 0.2) (layer "F.Cu") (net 13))
 (via (at 136.5 66.2) (size 0.6) (drill 0.3) (layers "F.Cu" "B.Cu") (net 13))
 (via (at 137.513777 67.339864) (size 0.6) (drill 0.3) (layers "F.Cu" "B.Cu") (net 13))
 (segment (start 136.5 66.326087) (end 137.513777 67.339864) (width 0.2) (layer "B.Cu") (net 13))
 (segment (start 136.5 66.2) (end 136.5 66.326087) (width 0.2) (layer "B.Cu") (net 13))
 (segment (start 139.548569 68.225) (end 139.552 68.221569) (width 0.35) (layer "F.Cu") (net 12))
 (segment (start 138.6625 68.225) (end 139.548569 68.225) (width 0.35) (layer "F.Cu") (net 12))
 (segment (start 141.848999 67.651001) (end 142.4 67.1) (width 0.35) (layer "F.Cu") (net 12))
 (segment (start 141.848999 68.1) (end 141.848999 67.651001) (width 0.35) (layer "F.Cu") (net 12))
 (via (at 139.552 68.221569) (size 0.6) (drill 0.3) (layers "F.Cu" "B.Cu") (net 12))
 (via (at 141.848999 68.1) (size 0.6) (drill 0.3) (layers "F.Cu" "B.Cu") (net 12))
 (segment (start 141.72743 68.221569) (end 141.848999 68.1) (width 0.35) (layer "B.Cu") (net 12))
 (segment (start 141.30517 68.221569) (end 141.72743 68.221569) (width 0.35) (layer "B.Cu") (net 12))
 (segment (start 139.552 68.221569) (end 141.30517 68.221569) (width 0.35) (layer "B.Cu") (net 12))
 (segment (start 131.22 64.5) (end 131.22 65.2075) (width 0.2) (layer "F.Cu") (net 5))
 (segment (start 131.22 65.2075) (end 132.9375 66.925) (width 0.2) (layer "F.Cu") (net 5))
 (segment (start 130.725 67.575) (end 130.5 67.8) (width 0.35) (layer "F.Cu") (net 4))
 (segment (start 132.9375 67.575) (end 130.725 67.575) (width 0.35) (layer "F.Cu") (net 4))
 (segment (start 130.5 70.549062) (end 130.5 70.7) (width 0.35) (layer "F.Cu") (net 6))
 (segment (start 132.174062 68.875) (end 130.5 70.549062) (width 0.35) (layer "F.Cu") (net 6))
 (segment (start 132.9375 68.875) (end 132.174062 68.875) (width 0.35) (layer "F.Cu") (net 6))
 (segment (start 138.462501 66.725001) (end 138.6625 66.925) (width 0.2) (layer "F.Cu") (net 14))
 (segment (start 137.203698 66.8) (end 137.278697 66.725001) (width 0.2) (layer "F.Cu") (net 14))
 (segment (start 133.76 64.5) (end 136.06 66.8) (width 0.2) (layer "F.Cu") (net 14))
 (segment (start 137.278697 66.725001) (end 138.462501 66.725001) (width 0.2) (layer "F.Cu") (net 14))
 (segment (start 136.06 66.8) (end 137.203698 66.8) (width 0.2) (layer "F.Cu") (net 14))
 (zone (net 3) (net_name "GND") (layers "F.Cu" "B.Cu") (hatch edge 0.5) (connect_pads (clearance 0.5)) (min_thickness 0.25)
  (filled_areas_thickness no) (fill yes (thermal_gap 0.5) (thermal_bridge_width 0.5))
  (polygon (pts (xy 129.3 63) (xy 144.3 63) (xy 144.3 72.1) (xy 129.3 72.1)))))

